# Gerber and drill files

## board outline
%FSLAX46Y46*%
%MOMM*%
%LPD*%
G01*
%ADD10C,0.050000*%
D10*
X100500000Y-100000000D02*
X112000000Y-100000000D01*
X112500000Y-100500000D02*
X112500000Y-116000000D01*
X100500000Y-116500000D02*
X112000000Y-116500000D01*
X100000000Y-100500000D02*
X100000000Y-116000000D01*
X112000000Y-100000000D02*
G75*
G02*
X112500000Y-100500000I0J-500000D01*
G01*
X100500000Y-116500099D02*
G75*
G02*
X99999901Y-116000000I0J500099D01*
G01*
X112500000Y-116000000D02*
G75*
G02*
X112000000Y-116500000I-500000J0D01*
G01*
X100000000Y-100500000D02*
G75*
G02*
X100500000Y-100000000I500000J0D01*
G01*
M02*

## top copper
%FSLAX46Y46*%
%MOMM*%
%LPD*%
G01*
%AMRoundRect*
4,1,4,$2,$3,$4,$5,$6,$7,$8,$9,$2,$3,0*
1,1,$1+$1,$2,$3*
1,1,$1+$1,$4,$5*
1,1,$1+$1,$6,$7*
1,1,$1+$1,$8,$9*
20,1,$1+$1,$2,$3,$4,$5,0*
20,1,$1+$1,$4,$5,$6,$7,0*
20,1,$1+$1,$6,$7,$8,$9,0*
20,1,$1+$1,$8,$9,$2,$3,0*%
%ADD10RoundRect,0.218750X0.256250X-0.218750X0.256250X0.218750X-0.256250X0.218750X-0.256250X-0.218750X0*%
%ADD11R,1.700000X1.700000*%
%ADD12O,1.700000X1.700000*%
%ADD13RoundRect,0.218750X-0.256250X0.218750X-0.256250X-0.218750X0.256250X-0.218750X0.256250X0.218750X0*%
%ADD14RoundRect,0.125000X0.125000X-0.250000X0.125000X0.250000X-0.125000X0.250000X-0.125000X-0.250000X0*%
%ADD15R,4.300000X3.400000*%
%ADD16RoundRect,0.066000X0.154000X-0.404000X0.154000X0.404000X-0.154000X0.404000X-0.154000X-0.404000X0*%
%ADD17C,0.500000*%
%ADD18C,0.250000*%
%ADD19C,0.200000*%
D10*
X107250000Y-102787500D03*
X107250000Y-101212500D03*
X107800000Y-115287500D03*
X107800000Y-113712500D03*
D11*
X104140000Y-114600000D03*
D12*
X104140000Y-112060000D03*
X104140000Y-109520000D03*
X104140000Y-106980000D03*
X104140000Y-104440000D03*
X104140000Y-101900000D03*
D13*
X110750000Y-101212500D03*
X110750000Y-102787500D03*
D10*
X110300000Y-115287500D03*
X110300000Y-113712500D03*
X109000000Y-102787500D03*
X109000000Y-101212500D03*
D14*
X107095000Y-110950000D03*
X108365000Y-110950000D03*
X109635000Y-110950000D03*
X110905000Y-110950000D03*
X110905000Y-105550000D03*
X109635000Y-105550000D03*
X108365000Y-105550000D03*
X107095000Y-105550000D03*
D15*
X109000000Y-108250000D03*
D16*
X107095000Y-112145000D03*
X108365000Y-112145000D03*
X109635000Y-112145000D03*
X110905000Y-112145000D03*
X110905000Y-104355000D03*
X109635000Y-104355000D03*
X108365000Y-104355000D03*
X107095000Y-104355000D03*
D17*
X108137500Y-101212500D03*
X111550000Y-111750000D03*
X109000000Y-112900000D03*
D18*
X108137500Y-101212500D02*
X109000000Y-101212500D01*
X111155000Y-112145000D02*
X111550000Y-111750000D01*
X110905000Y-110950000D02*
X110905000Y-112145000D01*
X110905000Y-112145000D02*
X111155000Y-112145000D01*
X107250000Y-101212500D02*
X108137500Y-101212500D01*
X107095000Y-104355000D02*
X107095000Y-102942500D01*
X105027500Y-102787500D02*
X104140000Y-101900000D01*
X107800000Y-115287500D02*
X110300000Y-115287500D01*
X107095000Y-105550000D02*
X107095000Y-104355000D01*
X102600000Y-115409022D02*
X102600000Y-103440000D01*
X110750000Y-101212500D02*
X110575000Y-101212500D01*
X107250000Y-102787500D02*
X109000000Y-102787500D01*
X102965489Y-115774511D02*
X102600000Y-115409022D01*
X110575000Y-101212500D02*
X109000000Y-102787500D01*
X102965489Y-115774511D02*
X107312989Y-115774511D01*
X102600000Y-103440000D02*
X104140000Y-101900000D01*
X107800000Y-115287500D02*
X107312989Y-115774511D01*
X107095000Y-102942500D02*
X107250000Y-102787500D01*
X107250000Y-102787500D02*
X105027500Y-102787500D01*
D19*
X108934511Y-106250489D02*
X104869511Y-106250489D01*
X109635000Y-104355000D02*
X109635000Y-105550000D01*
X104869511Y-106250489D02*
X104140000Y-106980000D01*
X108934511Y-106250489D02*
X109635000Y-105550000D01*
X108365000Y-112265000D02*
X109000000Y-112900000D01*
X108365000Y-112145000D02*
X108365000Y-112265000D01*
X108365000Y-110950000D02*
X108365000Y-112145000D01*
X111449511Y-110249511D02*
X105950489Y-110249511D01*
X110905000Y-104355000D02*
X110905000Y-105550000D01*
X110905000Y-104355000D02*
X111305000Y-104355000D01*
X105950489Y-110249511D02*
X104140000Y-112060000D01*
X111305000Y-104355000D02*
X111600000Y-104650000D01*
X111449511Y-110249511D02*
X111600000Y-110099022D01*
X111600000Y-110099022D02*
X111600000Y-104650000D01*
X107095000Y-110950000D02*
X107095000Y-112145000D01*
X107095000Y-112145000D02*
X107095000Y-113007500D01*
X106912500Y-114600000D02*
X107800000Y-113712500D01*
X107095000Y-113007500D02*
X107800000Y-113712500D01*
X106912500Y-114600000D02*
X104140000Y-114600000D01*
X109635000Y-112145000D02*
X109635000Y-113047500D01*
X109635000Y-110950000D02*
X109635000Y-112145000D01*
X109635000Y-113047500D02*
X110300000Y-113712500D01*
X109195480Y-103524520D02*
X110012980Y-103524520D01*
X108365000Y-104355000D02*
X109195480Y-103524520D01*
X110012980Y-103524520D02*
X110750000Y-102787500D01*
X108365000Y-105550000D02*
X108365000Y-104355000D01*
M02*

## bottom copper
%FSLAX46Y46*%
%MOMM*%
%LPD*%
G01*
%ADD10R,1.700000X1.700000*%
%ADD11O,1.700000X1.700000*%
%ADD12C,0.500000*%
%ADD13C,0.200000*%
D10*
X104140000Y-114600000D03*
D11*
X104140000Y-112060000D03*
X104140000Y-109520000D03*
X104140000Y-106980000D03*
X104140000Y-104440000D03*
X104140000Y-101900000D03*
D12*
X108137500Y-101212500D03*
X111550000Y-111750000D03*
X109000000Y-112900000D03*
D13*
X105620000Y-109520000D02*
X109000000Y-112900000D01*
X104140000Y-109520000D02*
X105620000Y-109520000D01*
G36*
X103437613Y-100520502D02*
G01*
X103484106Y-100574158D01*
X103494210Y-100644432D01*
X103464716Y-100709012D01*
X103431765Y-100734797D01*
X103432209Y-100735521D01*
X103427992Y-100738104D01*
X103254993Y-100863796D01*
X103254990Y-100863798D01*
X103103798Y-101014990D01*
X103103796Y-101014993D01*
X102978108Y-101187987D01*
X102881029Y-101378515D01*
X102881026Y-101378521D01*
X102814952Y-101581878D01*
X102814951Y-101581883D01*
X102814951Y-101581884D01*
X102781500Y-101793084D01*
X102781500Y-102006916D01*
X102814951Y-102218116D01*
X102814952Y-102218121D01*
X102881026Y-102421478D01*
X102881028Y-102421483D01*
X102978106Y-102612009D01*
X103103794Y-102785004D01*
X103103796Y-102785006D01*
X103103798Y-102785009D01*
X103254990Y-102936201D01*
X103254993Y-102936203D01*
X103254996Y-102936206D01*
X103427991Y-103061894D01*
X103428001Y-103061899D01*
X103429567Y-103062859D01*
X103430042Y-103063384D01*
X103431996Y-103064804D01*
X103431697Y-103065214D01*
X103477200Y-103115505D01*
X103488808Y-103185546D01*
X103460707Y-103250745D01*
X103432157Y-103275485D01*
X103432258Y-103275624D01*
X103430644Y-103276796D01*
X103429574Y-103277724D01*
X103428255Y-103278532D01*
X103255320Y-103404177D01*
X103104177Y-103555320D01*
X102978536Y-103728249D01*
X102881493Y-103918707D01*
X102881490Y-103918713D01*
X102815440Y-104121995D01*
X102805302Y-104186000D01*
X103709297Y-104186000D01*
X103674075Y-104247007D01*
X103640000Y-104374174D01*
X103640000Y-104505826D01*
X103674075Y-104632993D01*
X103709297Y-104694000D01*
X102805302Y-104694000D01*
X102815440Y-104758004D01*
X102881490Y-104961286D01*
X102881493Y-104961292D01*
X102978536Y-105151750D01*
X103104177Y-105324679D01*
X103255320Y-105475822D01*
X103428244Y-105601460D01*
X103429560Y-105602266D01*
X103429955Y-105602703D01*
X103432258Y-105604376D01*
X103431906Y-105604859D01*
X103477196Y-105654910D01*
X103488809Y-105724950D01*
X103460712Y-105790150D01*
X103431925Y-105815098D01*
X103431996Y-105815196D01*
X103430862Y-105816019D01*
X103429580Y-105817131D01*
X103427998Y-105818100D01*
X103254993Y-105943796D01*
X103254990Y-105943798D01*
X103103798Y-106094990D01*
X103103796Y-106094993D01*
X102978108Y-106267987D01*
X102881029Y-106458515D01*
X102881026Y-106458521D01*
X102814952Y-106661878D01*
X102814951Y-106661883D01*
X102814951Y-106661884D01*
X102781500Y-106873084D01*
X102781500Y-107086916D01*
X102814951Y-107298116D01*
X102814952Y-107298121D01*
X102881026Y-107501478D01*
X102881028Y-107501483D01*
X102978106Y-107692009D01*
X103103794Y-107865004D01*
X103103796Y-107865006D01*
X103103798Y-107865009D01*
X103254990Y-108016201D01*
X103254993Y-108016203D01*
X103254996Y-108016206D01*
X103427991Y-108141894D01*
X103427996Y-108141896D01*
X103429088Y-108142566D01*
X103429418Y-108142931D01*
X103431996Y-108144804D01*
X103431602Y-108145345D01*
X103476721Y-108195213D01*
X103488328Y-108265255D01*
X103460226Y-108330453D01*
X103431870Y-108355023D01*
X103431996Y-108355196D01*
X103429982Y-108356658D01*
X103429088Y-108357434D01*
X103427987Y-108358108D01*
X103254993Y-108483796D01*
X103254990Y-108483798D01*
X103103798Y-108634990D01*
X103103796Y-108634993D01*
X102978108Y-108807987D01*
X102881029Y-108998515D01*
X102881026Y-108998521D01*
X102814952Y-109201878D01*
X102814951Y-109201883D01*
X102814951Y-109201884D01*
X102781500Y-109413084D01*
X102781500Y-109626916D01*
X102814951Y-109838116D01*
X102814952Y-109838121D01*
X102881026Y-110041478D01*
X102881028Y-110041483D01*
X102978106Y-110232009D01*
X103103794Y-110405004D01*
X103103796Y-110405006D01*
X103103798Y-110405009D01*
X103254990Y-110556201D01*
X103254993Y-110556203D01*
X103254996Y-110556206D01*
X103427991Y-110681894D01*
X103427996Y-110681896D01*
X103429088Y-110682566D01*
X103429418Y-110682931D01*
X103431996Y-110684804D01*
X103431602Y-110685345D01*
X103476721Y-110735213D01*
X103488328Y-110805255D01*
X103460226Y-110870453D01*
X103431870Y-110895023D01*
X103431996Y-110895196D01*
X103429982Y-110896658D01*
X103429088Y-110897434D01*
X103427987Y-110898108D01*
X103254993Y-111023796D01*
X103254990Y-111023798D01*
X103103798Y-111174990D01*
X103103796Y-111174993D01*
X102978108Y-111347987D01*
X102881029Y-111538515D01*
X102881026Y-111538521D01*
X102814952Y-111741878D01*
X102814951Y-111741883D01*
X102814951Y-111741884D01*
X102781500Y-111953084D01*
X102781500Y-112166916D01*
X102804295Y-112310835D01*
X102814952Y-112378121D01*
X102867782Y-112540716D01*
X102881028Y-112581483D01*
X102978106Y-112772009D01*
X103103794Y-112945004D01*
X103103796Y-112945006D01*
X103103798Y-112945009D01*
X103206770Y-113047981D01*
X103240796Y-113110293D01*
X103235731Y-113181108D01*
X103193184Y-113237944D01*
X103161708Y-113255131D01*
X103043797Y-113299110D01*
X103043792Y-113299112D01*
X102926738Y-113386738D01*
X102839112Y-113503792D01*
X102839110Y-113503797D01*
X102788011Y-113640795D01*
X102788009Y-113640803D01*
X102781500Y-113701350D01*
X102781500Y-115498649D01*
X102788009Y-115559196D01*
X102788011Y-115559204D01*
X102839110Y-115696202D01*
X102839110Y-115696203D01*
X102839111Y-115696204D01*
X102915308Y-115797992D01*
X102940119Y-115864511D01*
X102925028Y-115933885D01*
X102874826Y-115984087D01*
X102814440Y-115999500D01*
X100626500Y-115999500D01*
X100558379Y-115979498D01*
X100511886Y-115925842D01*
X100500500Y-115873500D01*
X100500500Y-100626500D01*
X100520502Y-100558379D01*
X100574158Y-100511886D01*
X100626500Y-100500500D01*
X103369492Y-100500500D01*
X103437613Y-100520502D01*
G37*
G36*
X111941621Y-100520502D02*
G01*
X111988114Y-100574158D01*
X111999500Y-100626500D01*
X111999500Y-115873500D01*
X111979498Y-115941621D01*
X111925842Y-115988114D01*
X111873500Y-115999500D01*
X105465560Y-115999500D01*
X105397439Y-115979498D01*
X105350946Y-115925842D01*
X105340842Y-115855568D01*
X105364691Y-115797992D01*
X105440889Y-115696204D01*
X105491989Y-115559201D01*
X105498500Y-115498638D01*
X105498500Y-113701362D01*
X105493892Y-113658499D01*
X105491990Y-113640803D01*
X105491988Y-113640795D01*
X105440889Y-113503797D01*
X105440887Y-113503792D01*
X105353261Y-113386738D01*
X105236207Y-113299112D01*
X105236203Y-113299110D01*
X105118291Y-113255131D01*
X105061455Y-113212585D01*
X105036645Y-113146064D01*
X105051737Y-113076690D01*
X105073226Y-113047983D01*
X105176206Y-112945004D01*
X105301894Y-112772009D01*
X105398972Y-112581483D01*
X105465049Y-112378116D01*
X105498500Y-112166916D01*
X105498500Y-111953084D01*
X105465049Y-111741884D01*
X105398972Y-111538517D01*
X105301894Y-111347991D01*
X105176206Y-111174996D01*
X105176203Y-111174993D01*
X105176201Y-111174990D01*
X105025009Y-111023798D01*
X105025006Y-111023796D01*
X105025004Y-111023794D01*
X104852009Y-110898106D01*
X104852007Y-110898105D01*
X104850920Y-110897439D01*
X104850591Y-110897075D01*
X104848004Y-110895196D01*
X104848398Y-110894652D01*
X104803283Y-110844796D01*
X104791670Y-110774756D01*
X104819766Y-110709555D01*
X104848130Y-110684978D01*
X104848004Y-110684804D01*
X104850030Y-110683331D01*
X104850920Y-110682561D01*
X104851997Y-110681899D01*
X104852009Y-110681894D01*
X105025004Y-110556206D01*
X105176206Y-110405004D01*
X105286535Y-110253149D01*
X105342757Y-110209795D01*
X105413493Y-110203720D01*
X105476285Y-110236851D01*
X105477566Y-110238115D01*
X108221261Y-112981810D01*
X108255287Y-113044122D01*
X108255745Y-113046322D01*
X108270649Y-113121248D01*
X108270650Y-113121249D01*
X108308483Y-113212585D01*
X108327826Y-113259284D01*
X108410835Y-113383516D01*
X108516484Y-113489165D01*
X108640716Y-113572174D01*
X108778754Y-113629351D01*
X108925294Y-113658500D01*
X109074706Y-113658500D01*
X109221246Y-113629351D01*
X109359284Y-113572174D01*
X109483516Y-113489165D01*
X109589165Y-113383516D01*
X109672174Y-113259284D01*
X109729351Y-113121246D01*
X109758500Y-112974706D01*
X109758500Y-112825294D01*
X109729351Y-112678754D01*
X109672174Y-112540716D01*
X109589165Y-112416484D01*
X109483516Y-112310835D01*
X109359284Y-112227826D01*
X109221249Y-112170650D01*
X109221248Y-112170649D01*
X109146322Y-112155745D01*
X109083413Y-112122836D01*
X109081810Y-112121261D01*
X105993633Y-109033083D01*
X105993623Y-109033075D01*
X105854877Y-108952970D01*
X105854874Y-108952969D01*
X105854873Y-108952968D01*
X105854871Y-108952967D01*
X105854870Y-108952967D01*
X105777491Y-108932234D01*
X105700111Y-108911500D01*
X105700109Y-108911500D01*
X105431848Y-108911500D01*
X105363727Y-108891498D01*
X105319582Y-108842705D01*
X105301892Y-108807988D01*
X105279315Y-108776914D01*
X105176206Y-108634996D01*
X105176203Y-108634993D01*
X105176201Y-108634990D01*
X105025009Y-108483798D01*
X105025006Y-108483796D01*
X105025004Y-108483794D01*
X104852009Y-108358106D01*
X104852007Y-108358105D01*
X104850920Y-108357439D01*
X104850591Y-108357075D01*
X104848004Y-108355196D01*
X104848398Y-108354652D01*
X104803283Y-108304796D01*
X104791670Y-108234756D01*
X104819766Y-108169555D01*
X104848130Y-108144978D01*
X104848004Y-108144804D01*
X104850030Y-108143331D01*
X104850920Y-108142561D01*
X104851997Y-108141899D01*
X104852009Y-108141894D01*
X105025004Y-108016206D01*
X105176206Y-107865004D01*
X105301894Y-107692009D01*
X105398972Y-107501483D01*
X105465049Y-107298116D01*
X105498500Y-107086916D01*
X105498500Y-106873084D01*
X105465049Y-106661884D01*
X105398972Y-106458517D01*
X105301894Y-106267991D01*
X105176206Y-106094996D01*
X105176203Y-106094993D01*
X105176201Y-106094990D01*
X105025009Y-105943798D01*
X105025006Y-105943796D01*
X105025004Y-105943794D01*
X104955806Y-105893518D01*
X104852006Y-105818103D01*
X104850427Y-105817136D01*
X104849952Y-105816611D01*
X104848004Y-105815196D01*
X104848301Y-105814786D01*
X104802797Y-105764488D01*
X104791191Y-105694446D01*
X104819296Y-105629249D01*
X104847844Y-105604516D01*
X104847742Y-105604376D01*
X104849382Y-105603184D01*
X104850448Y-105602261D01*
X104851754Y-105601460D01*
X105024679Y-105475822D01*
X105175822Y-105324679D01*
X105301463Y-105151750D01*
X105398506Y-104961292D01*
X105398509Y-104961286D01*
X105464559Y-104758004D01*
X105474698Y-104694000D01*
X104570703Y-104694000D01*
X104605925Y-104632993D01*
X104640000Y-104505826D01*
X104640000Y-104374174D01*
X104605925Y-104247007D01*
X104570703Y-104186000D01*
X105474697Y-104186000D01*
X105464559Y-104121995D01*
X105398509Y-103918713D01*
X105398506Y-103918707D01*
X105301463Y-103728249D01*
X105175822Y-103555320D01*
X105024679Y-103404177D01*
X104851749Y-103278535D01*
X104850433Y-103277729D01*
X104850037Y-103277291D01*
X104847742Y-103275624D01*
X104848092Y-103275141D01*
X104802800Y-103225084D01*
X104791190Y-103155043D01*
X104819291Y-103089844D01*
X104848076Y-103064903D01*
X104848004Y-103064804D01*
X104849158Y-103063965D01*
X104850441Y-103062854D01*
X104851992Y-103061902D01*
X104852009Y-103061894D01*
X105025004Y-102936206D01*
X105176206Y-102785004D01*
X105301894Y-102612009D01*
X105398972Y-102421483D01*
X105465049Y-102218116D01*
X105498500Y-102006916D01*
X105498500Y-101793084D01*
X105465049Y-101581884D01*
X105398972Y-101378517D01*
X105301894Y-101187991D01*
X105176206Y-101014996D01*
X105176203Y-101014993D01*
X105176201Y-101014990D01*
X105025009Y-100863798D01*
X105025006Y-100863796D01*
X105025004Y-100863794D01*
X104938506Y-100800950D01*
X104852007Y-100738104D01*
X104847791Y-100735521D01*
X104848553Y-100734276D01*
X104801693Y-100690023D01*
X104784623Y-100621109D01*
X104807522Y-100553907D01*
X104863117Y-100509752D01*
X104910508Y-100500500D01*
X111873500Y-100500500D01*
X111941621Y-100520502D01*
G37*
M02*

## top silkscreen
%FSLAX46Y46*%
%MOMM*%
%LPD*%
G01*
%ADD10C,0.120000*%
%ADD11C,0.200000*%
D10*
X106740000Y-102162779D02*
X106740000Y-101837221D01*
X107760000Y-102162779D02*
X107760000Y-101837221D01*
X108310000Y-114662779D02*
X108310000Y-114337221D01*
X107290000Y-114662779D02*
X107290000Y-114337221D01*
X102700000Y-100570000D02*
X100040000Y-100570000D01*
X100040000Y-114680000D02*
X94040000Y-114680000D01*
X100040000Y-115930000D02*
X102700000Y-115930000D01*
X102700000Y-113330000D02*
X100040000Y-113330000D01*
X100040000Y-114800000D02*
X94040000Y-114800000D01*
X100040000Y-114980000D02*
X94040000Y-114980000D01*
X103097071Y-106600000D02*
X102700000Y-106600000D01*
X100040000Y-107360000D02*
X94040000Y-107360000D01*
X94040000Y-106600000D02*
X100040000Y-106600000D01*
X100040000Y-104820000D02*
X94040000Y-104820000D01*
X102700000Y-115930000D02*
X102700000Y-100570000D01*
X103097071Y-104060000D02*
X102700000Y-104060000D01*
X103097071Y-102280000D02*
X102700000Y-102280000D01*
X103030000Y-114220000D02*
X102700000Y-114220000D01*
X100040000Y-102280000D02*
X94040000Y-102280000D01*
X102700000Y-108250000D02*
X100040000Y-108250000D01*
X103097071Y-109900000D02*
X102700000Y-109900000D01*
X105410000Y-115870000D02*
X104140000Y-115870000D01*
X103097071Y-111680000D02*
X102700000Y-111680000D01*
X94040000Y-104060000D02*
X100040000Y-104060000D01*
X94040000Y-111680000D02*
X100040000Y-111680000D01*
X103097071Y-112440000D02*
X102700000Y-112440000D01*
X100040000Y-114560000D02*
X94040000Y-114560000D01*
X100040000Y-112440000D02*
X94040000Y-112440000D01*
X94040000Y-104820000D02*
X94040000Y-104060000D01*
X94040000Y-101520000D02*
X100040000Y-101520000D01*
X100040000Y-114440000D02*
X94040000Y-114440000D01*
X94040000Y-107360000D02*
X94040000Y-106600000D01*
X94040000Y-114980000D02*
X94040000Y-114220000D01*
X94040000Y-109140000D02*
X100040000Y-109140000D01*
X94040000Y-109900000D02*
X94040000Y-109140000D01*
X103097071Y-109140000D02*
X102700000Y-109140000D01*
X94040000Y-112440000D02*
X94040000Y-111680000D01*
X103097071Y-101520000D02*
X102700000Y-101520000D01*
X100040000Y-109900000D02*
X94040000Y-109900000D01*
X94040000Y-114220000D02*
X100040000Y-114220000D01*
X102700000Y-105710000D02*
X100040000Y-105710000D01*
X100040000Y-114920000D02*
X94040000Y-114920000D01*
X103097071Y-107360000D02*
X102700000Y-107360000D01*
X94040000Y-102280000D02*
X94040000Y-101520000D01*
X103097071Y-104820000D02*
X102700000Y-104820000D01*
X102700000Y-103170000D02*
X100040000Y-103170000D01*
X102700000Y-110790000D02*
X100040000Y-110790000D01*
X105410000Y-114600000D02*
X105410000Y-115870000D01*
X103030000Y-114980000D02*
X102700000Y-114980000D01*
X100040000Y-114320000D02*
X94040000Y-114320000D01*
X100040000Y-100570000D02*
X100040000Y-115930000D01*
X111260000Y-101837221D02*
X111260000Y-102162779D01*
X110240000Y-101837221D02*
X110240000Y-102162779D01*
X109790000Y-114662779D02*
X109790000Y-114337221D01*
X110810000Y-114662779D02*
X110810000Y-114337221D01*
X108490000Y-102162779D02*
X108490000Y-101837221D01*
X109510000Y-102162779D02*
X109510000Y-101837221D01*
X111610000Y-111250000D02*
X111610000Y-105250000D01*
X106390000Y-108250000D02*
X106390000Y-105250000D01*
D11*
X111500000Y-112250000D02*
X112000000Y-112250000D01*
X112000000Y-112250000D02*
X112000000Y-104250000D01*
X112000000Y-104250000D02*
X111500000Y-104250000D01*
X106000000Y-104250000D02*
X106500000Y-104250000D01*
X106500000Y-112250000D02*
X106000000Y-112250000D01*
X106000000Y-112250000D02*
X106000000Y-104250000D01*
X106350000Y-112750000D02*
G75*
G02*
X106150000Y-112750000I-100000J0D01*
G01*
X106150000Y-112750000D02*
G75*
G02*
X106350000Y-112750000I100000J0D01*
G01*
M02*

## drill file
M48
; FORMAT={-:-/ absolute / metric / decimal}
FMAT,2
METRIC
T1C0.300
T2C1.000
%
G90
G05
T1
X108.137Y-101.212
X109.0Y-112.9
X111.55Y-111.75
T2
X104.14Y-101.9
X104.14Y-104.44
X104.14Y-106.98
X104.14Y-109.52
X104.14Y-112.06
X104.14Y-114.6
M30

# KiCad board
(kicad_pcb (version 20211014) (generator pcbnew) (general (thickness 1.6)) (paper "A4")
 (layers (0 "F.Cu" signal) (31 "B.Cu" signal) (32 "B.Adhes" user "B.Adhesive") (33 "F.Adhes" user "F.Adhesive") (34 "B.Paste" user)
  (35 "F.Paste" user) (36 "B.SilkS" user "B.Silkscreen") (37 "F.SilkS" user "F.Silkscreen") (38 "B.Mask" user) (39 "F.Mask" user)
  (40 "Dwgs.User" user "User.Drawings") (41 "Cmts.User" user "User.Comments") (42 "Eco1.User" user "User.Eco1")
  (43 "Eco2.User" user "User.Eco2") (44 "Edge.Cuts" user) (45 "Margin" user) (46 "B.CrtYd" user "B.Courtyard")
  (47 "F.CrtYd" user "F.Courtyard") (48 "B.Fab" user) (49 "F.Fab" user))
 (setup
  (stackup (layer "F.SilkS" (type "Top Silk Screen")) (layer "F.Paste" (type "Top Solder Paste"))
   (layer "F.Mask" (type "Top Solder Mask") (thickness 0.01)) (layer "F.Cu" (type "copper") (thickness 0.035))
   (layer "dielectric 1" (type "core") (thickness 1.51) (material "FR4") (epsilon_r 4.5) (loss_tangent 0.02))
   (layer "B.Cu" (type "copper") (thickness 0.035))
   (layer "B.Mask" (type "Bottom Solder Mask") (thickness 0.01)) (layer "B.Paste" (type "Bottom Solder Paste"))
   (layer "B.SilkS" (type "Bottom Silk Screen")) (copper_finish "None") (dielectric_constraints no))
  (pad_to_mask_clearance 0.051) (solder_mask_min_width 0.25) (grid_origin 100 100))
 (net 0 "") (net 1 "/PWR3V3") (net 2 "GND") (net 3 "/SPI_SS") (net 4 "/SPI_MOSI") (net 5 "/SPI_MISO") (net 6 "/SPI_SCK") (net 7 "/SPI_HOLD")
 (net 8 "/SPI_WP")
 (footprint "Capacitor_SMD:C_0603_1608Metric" (layer "F.Cu") (at 107.25 102 90)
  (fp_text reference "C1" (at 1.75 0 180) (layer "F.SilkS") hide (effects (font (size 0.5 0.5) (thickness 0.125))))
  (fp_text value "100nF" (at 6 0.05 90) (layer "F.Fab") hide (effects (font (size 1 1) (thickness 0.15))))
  (fp_line (start -0.162779 -0.51) (end 0.162779 -0.51) (layer "F.SilkS") (width 0.12))
  (fp_line (start -0.162779 0.51) (end 0.162779 0.51) (layer "F.SilkS") (width 0.12))
  (pad "1" smd roundrect locked (at -0.7875 0 90) (size 0.875 0.95) (layers "F.Cu" "F.Paste" "F.Mask") (roundrect_rratio 0.25)
   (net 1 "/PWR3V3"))
  (pad "2" smd roundrect locked (at 0.7875 0 90) (size 0.875 0.95) (layers "F.Cu" "F.Paste" "F.Mask") (roundrect_rratio 0.25) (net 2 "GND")))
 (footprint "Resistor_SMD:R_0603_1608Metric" (layer "F.Cu") (at 107.8 114.5 90)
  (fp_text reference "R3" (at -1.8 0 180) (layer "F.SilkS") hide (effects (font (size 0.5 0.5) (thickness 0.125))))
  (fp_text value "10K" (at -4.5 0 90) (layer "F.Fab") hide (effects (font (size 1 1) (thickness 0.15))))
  (fp_line (start -0.162779 0.51) (end 0.162779 0.51) (layer "F.SilkS") (width 0.12))
  (fp_line (start -0.162779 -0.51) (end 0.162779 -0.51) (layer "F.SilkS") (width 0.12))
  (pad "1" smd roundrect locked (at -0.7875 0 90) (size 0.875 0.95) (layers "F.Cu" "F.Paste" "F.Mask") (roundrect_rratio 0.25)
   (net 1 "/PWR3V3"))
  (pad "2" smd roundrect locked (at 0.7875 0 90) (size 0.875 0.95) (layers "F.Cu" "F.Paste" "F.Mask") (roundrect_rratio 0.25)
   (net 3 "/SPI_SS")))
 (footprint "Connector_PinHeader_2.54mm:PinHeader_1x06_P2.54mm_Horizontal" (layer "F.Cu") (at 104.14 114.6 180)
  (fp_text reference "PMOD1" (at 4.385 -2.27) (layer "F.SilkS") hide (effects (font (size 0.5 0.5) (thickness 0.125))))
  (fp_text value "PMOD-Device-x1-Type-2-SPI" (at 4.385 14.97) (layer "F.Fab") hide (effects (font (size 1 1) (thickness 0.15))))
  (fp_line (start 1.44 14.03) (end 4.1 14.03) (layer "F.SilkS") (width 0.12))
  (fp_line (start 4.1 -0.08) (end 10.1 -0.08) (layer "F.SilkS") (width 0.12))
  (fp_line (start 4.1 -1.33) (end 1.44 -1.33) (layer "F.SilkS") (width 0.12))
  (fp_line (start 1.44 1.27) (end 4.1 1.27) (layer "F.SilkS") (width 0.12))
  (fp_line (start 4.1 -0.2) (end 10.1 -0.2) (layer "F.SilkS") (width 0.12))
  (fp_line (start 4.1 -0.38) (end 10.1 -0.38) (layer "F.SilkS") (width 0.12))
  (fp_line (start 1.042929 8) (end 1.44 8) (layer "F.SilkS") (width 0.12))
  (fp_line (start 4.1 7.24) (end 10.1 7.24) (layer "F.SilkS") (width 0.12))
  (fp_line (start 10.1 8) (end 4.1 8) (layer "F.SilkS") (width 0.12))
  (fp_line (start 4.1 9.78) (end 10.1 9.78) (layer "F.SilkS") (width 0.12))
  (fp_line (start 1.44 -1.33) (end 1.44 14.03) (layer "F.SilkS") (width 0.12))
  (fp_line (start 1.042929 10.54) (end 1.44 10.54) (layer "F.SilkS") (width 0.12))
  (fp_line (start 1.042929 12.32) (end 1.44 12.32) (layer "F.SilkS") (width 0.12))
  (fp_line (start 1.11 0.38) (end 1.44 0.38) (layer "F.SilkS") (width 0.12))
  (fp_line (start 4.1 12.32) (end 10.1 12.32) (layer "F.SilkS") (width 0.12))
  (fp_line (start 1.44 6.35) (end 4.1 6.35) (layer "F.SilkS") (width 0.12))
  (fp_line (start 1.042929 4.7) (end 1.44 4.7) (layer "F.SilkS") (width 0.12))
  (fp_line (start -1.27 -1.27) (end 0 -1.27) (layer "F.SilkS") (width 0.12))
  (fp_line (start 1.042929 2.92) (end 1.44 2.92) (layer "F.SilkS") (width 0.12))
  (fp_line (start 10.1 10.54) (end 4.1 10.54) (layer "F.SilkS") (width 0.12))
  (fp_line (start 10.1 2.92) (end 4.1 2.92) (layer "F.SilkS") (width 0.12))
  (fp_line (start 1.042929 2.16) (end 1.44 2.16) (layer "F.SilkS") (width 0.12))
  (fp_line (start 4.1 0.04) (end 10.1 0.04) (layer "F.SilkS") (width 0.12))
  (fp_line (start 4.1 2.16) (end 10.1 2.16) (layer "F.SilkS") (width 0.12))
  (fp_line (start 10.1 9.78) (end 10.1 10.54) (layer "F.SilkS") (width 0.12))
  (fp_line (start 10.1 13.08) (end 4.1 13.08) (layer "F.SilkS") (width 0.12))
  (fp_line (start 4.1 0.16) (end 10.1 0.16) (layer "F.SilkS") (width 0.12))
  (fp_line (start 10.1 7.24) (end 10.1 8) (layer "F.SilkS") (width 0.12))
  (fp_line (start 10.1 -0.38) (end 10.1 0.38) (layer "F.SilkS") (width 0.12))
  (fp_line (start 10.1 5.46) (end 4.1 5.46) (layer "F.SilkS") (width 0.12))
  (fp_line (start 10.1 4.7) (end 10.1 5.46) (layer "F.SilkS") (width 0.12))
  (fp_line (start 1.042929 5.46) (end 1.44 5.46) (layer "F.SilkS") (width 0.12))
  (fp_line (start 10.1 2.16) (end 10.1 2.92) (layer "F.SilkS") (width 0.12))
  (fp_line (start 1.042929 13.08) (end 1.44 13.08) (layer "F.SilkS") (width 0.12))
  (fp_line (start 4.1 4.7) (end 10.1 4.7) (layer "F.SilkS") (width 0.12))
  (fp_line (start 10.1 0.38) (end 4.1 0.38) (layer "F.SilkS") (width 0.12))
  (fp_line (start 1.44 8.89) (end 4.1 8.89) (layer "F.SilkS") (width 0.12))
  (fp_line (start 4.1 -0.32) (end 10.1 -0.32) (layer "F.SilkS") (width 0.12))
  (fp_line (start 1.042929 7.24) (end 1.44 7.24) (layer "F.SilkS") (width 0.12))
  (fp_line (start 10.1 12.32) (end 10.1 13.08) (layer "F.SilkS") (width 0.12))
  (fp_line (start 1.042929 9.78) (end 1.44 9.78) (layer "F.SilkS") (width 0.12))
  (fp_line (start 1.44 11.43) (end 4.1 11.43) (layer "F.SilkS") (width 0.12))
  (fp_line (start 1.44 3.81) (end 4.1 3.81) (layer "F.SilkS") (width 0.12))
  (fp_line (start -1.27 0) (end -1.27 -1.27) (layer "F.SilkS") (width 0.12))
  (fp_line (start 1.11 -0.38) (end 1.44 -0.38) (layer "F.SilkS") (width 0.12))
  (fp_line (start 4.1 0.28) (end 10.1 0.28) (layer "F.SilkS") (width 0.12))
  (fp_line (start 4.1 14.03) (end 4.1 -1.33) (layer "F.SilkS") (width 0.12))
  (pad "1" thru_hole rect locked (at 0 0 180) (size 1.7 1.7) (drill 1) (layers *.Cu *.Mask) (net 3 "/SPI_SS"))
  (pad "2" thru_hole oval locked (at 0 2.54 180) (size 1.7 1.7) (drill 1) (layers *.Cu *.Mask) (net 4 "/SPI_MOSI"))
  (pad "3" thru_hole oval locked (at 0 5.08 180) (size 1.7 1.7) (drill 1) (layers *.Cu *.Mask) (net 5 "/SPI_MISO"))
  (pad "4" thru_hole oval locked (at 0 7.62 180) (size 1.7 1.7) (drill 1) (layers *.Cu *.Mask) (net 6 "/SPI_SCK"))
  (pad "5" thru_hole oval locked (at 0 10.16 180) (size 1.7 1.7) (drill 1) (layers *.Cu *.Mask) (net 2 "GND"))
  (pad "6" thru_hole oval locked (at 0 12.7 180) (size 1.7 1.7) (drill 1) (layers *.Cu *.Mask) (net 1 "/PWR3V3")))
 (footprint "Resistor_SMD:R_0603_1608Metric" (layer "F.Cu") (at 110.75 102 -90)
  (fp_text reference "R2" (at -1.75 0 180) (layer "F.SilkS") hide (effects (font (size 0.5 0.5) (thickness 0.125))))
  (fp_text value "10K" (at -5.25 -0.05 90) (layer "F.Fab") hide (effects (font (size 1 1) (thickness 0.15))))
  (fp_line (start -0.162779 -0.51) (end 0.162779 -0.51) (layer "F.SilkS") (width 0.12))
  (fp_line (start -0.162779 0.51) (end 0.162779 0.51) (layer "F.SilkS") (width 0.12))
  (pad "1" smd roundrect locked (at -0.7875 0 270) (size 0.875 0.95) (layers "F.Cu" "F.Paste" "F.Mask") (roundrect_rratio 0.25)
   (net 1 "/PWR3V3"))
  (pad "2" smd roundrect locked (at 0.7875 0 270) (size 0.875 0.95) (layers "F.Cu" "F.Paste" "F.Mask") (roundrect_rratio 0.25)
   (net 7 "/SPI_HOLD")))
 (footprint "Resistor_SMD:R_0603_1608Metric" (layer "F.Cu") (at 110.3 114.5 90)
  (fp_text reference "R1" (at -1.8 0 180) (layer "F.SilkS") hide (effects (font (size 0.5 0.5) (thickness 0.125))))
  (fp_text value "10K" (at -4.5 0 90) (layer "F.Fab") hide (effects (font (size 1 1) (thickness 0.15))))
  (fp_line (start -0.162779 -0.51) (end 0.162779 -0.51) (layer "F.SilkS") (width 0.12))
  (fp_line (start -0.162779 0.51) (end 0.162779 0.51) (layer "F.SilkS") (width 0.12))
  (pad "1" smd roundrect locked (at -0.7875 0 90) (size 0.875 0.95) (layers "F.Cu" "F.Paste" "F.Mask") (roundrect_rratio 0.25)
   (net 1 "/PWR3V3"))
  (pad "2" smd roundrect locked (at 0.7875 0 90) (size 0.875 0.95) (layers "F.Cu" "F.Paste" "F.Mask") (roundrect_rratio 0.25)
   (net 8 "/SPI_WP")))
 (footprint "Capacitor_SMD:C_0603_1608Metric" (layer "F.Cu") (at 109 102 90)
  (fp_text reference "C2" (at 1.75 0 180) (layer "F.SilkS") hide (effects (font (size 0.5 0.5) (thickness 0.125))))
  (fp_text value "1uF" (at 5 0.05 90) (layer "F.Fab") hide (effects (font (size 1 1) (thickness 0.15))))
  (fp_line (start -0.162779 -0.51) (end 0.162779 -0.51) (layer "F.SilkS") (width 0.12))
  (fp_line (start -0.162779 0.51) (end 0.162779 0.51) (layer "F.SilkS") (width 0.12))
  (pad "1" smd roundrect locked (at -0.7875 0 90) (size 0.875 0.95) (layers "F.Cu" "F.Paste" "F.Mask") (roundrect_rratio 0.25)
   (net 1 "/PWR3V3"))
  (pad "2" smd roundrect locked (at 0.7875 0 90) (size 0.875 0.95) (layers "F.Cu" "F.Paste" "F.Mask") (roundrect_rratio 0.25) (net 2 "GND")))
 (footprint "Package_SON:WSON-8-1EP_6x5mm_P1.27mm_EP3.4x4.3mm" (layer "F.Cu") (at 109 108.25 90)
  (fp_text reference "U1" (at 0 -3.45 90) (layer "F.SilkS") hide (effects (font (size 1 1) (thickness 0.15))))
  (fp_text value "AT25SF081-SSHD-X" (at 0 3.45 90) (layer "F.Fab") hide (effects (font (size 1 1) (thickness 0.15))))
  (fp_line (start -3 2.61) (end 3 2.61) (layer "F.SilkS") (width 0.12))
  (fp_line (start 0 -2.61) (end 3 -2.61) (layer "F.SilkS") (width 0.12))
  (pad "" smd roundrect (at -0.85 1.075 90) (size 1.37 1.73) (layers "F.Paste") (roundrect_rratio 0.182482))
  (pad "" smd roundrect (at 0.85 -1.075 90) (size 1.37 1.73) (layers "F.Paste") (roundrect_rratio 0.182482))
  (pad "" smd roundrect (at -0.85 -1.075 90) (size 1.37 1.73) (layers "F.Paste") (roundrect_rratio 0.182482))
  (pad "" smd roundrect (at 0.85 1.075 90) (size 1.37 1.73) (layers "F.Paste") (roundrect_rratio 0.182482))
  (pad "1" smd roundrect (at -2.7 -1.905 90) (size 0.75 0.5) (layers "F.Cu" "F.Paste" "F.Mask") (roundrect_rratio 0.25) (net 3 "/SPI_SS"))
  (pad "2" smd roundrect (at -2.7 -0.635 90) (size 0.75 0.5) (layers "F.Cu" "F.Paste" "F.Mask") (roundrect_rratio 0.25) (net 5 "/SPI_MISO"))
  (pad "3" smd roundrect (at -2.7 0.635 90) (size 0.75 0.5) (layers "F.Cu" "F.Paste" "F.Mask") (roundrect_rratio 0.25) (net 8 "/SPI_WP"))
  (pad "4" smd roundrect (at -2.7 1.905 90) (size 0.75 0.5) (layers "F.Cu" "F.Paste" "F.Mask") (roundrect_rratio 0.25) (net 2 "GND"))
  (pad "5" smd roundrect (at 2.7 1.905 90) (size 0.75 0.5) (layers "F.Cu" "F.Paste" "F.Mask") (roundrect_rratio 0.25) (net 4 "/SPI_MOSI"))
  (pad "6" smd roundrect (at 2.7 0.635 90) (size 0.75 0.5) (layers "F.Cu" "F.Paste" "F.Mask") (roundrect_rratio 0.25) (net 6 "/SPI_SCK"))
  (pad "7" smd roundrect (at 2.7 -0.635 90) (size 0.75 0.5) (layers "F.Cu" "F.Paste" "F.Mask") (roundrect_rratio 0.25) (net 7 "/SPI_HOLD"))
  (pad "8" smd roundrect (at 2.7 -1.905 90) (size 0.75 0.5) (layers "F.Cu" "F.Paste" "F.Mask") (roundrect_rratio 0.25) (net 1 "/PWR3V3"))
  (pad "9" smd rect (at 0 0 90) (size 3.4 4.3) (layers "F.Cu" "F.Mask")))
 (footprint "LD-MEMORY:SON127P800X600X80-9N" (layer "F.Cu") (at 109 108.25 90)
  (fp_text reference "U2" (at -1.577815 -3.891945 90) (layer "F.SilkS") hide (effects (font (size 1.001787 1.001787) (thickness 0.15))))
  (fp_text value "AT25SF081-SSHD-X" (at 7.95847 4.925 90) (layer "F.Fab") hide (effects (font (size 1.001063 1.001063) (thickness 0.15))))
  (fp_line (start -4 2.5) (end -4 3) (layer "F.SilkS") (width 0.2))
  (fp_line (start -4 3) (end 4 3) (layer "F.SilkS") (width 0.2))
  (fp_line (start 4 3) (end 4 2.5) (layer "F.SilkS") (width 0.2))
  (fp_line (start 4 -3) (end 4 -2.5) (layer "F.SilkS") (width 0.2))
  (fp_line (start -4 -2.5) (end -4 -3) (layer "F.SilkS") (width 0.2))
  (fp_line (start -4 -3) (end 4 -3) (layer "F.SilkS") (width 0.2))
  (fp_circle (center -4.5 -2.75) (end -4.4 -2.75) (layer "F.SilkS") (width 0.2) (fill none))
  (pad "1" smd roundrect (at -3.895 -1.905 90) (size 0.94 0.44) (layers "F.Cu" "F.Paste" "F.Mask") (roundrect_rratio 0.15) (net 3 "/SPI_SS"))
  (pad "2" smd roundrect (at -3.895 -0.635 90) (size 0.94 0.44) (layers "F.Cu" "F.Paste" "F.Mask") (roundrect_rratio 0.15)
   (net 5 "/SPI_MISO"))
  (pad "3" smd roundrect (at -3.895 0.635 90) (size 0.94 0.44) (layers "F.Cu" "F.Paste" "F.Mask") (roundrect_rratio 0.15) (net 8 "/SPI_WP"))
  (pad "4" smd roundrect (at -3.895 1.905 90) (size 0.94 0.44) (layers "F.Cu" "F.Paste" "F.Mask") (roundrect_rratio 0.15) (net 2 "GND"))
  (pad "5" smd roundrect (at 3.895 1.905 90) (size 0.94 0.44) (layers "F.Cu" "F.Paste" "F.Mask") (roundrect_rratio 0.15) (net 4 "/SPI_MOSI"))
  (pad "6" smd roundrect (at 3.895 0.635 90) (size 0.94 0.44) (layers "F.Cu" "F.Paste" "F.Mask") (roundrect_rratio 0.15) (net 6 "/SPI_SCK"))
  (pad "7" smd roundrect (at 3.895 -0.635 90) (size 0.94 0.44) (layers "F.Cu" "F.Paste" "F.Mask") (roundrect_rratio 0.15)
   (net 7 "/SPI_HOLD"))
  (pad "8" smd roundrect (at 3.895 -1.905 90) (size 0.94 0.44) (layers "F.Cu" "F.Paste" "F.Mask") (roundrect_rratio 0.15) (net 1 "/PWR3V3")))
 (gr_line (start 100.5 100) (end 112 100) (layer "Edge.Cuts") (width 0.05))
 (gr_line (start 112.5 100.5) (end 112.5 116) (layer "Edge.Cuts") (width 0.05))
 (gr_line (start 100.5 116.5) (end 112 116.5) (layer "Edge.Cuts") (width 0.05))
 (gr_line (start 100 100.5) (end 100 116) (layer "Edge.Cuts") (width 0.05))
 (gr_arc (start 112 100) (mid 112.353553 100.146447) (end 112.5 100.5) (layer "Edge.Cuts") (width 0.05))
 (gr_arc (start 100.5 116.500099) (mid 100.146377 116.353623) (end 99.999901 116) (layer "Edge.Cuts") (width 0.05))
 (gr_arc (start 112.5 116) (mid 112.353553 116.353553) (end 112 116.5) (layer "Edge.Cuts") (width 0.05))
 (gr_arc (start 100 100.5) (mid 100.146447 100.146447) (end 100.5 100) (layer "Edge.Cuts") (width 0.05))
 (segment (start 108.1375 101.2125) (end 109 101.2125) (width 0.25) (layer "F.Cu") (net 2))
 (segment (start 111.155 112.145) (end 111.55 111.75) (width 0.25) (layer "F.Cu") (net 2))
 (segment (start 110.905 110.95) (end 110.905 112.145) (width 0.25) (layer "F.Cu") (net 2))
 (segment (start 110.905 112.145) (end 111.155 112.145) (width 0.25) (layer "F.Cu") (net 2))
 (segment (start 107.25 101.2125) (end 108.1375 101.2125) (width 0.25) (layer "F.Cu") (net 2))
 (via (at 108.1375 101.2125) (size 0.5) (drill 0.3) (layers "F.Cu" "B.Cu") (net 2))
 (via (at 111.55 111.75) (size 0.5) (drill 0.3) (layers "F.Cu" "B.Cu") (free) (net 2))
 (segment (start 107.095 104.355) (end 107.095 102.9425) (width 0.25) (layer "F.Cu") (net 1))
 (segment (start 105.0275 102.7875) (end 104.14 101.9) (width 0.25) (layer "F.Cu") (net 1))
 (segment (start 107.8 115.2875) (end 110.3 115.2875) (width 0.25) (layer "F.Cu") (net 1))
 (segment (start 107.095 105.55) (end 107.095 104.355) (width 0.25) (layer "F.Cu") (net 1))
 (segment (start 102.6 115.409022) (end 102.6 103.44) (width 0.25) (layer "F.Cu") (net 1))
 (segment (start 110.75 101.2125) (end 110.575 101.2125) (width 0.25) (layer "F.Cu") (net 1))
 (segment (start 107.25 102.7875) (end 109 102.7875) (width 0.25) (layer "F.Cu") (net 1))
 (segment (start 102.965489 115.774511) (end 102.6 115.409022) (width 0.25) (layer "F.Cu") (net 1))
 (segment (start 110.575 101.2125) (end 109 102.7875) (width 0.25) (layer "F.Cu") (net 1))
 (segment (start 102.965489 115.774511) (end 107.312989 115.774511) (width 0.25) (layer "F.Cu") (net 1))
 (segment (start 102.6 103.44) (end 104.14 101.9) (width 0.25) (layer "F.Cu") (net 1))
 (segment (start 107.8 115.2875) (end 107.312989 115.774511) (width 0.25) (layer "F.Cu") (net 1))
 (segment (start 107.095 102.9425) (end 107.25 102.7875) (width 0.25) (layer "F.Cu") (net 1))
 (segment (start 107.25 102.7875) (end 105.0275 102.7875) (width 0.25) (layer "F.Cu") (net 1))
 (segment (start 108.934511 106.250489) (end 104.869511 106.250489) (width 0.2) (layer "F.Cu") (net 6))
 (segment (start 109.635 104.355) (end 109.635 105.55) (width 0.2) (layer "F.Cu") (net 6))
 (segment (start 104.869511 106.250489) (end 104.14 106.98) (width 0.2) (layer "F.Cu") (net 6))
 (segment (start 108.934511 106.250489) (end 109.635 105.55) (width 0.2) (layer "F.Cu") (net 6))
 (segment (start 108.365 112.265) (end 109 112.9) (width 0.2) (layer "F.Cu") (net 5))
 (segment (start 108.365 112.145) (end 108.365 112.265) (width 0.2) (layer "F.Cu") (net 5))
 (segment (start 108.365 110.95) (end 108.365 112.145) (width 0.2) (layer "F.Cu") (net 5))
 (via (at 109 112.9) (size 0.5) (drill 0.3) (layers "F.Cu" "B.Cu") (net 5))
 (segment (start 105.62 109.52) (end 109 112.9) (width 0.2) (layer "B.Cu") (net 5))
 (segment (start 104.14 109.52) (end 105.62 109.52) (width 0.2) (layer "B.Cu") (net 5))
 (segment (start 111.449511 110.249511) (end 105.950489 110.249511) (width 0.2) (layer "F.Cu") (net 4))
 (segment (start 110.905 104.355) (end 110.905 105.55) (width 0.2) (layer "F.Cu") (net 4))
 (segment (start 110.905 104.355) (end 111.305 104.355) (width 0.2) (layer "F.Cu") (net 4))
 (segment (start 105.950489 110.249511) (end 104.14 112.06) (width 0.2) (layer "F.Cu") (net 4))
 (segment (start 111.305 104.355) (end 111.6 104.65) (width 0.2) (layer "F.Cu") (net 4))
 (segment (start 111.449511 110.249511) (end 111.6 110.099022) (width 0.2) (layer "F.Cu") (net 4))
 (segment (start 111.6 110.099022) (end 111.6 104.65) (width 0.2) (layer "F.Cu") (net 4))
 (segment (start 107.095 110.95) (end 107.095 112.145) (width 0.2) (layer "F.Cu") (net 3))
 (segment (start 107.095 112.145) (end 107.095 113.0075) (width 0.2) (layer "F.Cu") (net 3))
 (segment (start 106.9125 114.6) (end 107.8 113.7125) (width 0.2) (layer "F.Cu") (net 3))
 (segment (start 107.095 113.0075) (end 107.8 113.7125) (width 0.2) (layer "F.Cu") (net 3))
 (segment (start 106.9125 114.6) (end 104.14 114.6) (width 0.2) (layer "F.Cu") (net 3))
 (segment (start 109.635 112.145) (end 109.635 113.0475) (width 0.2) (layer "F.Cu") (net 8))
 (segment (start 109.635 110.95) (end 109.635 112.145) (width 0.2) (layer "F.Cu") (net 8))
 (segment (start 109.635 113.0475) (end 110.3 113.7125) (width 0.2) (layer "F.Cu") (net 8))
 (segment (start 109.19548 103.52452) (end 110.01298 103.52452) (width 0.2) (layer "F.Cu") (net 7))
 (segment (start 108.365 104.355) (end 109.19548 103.52452) (width 0.2) (layer "F.Cu") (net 7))
 (segment (start 110.01298 103.52452) (end 110.75 102.7875) (width 0.2) (layer "F.Cu") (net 7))
 (segment (start 108.365 105.55) (end 108.365 104.355) (width 0.2) (layer "F.Cu") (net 7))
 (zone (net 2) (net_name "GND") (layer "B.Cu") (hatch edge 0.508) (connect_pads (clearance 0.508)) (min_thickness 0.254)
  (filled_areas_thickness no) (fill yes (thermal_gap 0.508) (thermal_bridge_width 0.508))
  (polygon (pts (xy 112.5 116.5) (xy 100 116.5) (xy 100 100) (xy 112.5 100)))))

